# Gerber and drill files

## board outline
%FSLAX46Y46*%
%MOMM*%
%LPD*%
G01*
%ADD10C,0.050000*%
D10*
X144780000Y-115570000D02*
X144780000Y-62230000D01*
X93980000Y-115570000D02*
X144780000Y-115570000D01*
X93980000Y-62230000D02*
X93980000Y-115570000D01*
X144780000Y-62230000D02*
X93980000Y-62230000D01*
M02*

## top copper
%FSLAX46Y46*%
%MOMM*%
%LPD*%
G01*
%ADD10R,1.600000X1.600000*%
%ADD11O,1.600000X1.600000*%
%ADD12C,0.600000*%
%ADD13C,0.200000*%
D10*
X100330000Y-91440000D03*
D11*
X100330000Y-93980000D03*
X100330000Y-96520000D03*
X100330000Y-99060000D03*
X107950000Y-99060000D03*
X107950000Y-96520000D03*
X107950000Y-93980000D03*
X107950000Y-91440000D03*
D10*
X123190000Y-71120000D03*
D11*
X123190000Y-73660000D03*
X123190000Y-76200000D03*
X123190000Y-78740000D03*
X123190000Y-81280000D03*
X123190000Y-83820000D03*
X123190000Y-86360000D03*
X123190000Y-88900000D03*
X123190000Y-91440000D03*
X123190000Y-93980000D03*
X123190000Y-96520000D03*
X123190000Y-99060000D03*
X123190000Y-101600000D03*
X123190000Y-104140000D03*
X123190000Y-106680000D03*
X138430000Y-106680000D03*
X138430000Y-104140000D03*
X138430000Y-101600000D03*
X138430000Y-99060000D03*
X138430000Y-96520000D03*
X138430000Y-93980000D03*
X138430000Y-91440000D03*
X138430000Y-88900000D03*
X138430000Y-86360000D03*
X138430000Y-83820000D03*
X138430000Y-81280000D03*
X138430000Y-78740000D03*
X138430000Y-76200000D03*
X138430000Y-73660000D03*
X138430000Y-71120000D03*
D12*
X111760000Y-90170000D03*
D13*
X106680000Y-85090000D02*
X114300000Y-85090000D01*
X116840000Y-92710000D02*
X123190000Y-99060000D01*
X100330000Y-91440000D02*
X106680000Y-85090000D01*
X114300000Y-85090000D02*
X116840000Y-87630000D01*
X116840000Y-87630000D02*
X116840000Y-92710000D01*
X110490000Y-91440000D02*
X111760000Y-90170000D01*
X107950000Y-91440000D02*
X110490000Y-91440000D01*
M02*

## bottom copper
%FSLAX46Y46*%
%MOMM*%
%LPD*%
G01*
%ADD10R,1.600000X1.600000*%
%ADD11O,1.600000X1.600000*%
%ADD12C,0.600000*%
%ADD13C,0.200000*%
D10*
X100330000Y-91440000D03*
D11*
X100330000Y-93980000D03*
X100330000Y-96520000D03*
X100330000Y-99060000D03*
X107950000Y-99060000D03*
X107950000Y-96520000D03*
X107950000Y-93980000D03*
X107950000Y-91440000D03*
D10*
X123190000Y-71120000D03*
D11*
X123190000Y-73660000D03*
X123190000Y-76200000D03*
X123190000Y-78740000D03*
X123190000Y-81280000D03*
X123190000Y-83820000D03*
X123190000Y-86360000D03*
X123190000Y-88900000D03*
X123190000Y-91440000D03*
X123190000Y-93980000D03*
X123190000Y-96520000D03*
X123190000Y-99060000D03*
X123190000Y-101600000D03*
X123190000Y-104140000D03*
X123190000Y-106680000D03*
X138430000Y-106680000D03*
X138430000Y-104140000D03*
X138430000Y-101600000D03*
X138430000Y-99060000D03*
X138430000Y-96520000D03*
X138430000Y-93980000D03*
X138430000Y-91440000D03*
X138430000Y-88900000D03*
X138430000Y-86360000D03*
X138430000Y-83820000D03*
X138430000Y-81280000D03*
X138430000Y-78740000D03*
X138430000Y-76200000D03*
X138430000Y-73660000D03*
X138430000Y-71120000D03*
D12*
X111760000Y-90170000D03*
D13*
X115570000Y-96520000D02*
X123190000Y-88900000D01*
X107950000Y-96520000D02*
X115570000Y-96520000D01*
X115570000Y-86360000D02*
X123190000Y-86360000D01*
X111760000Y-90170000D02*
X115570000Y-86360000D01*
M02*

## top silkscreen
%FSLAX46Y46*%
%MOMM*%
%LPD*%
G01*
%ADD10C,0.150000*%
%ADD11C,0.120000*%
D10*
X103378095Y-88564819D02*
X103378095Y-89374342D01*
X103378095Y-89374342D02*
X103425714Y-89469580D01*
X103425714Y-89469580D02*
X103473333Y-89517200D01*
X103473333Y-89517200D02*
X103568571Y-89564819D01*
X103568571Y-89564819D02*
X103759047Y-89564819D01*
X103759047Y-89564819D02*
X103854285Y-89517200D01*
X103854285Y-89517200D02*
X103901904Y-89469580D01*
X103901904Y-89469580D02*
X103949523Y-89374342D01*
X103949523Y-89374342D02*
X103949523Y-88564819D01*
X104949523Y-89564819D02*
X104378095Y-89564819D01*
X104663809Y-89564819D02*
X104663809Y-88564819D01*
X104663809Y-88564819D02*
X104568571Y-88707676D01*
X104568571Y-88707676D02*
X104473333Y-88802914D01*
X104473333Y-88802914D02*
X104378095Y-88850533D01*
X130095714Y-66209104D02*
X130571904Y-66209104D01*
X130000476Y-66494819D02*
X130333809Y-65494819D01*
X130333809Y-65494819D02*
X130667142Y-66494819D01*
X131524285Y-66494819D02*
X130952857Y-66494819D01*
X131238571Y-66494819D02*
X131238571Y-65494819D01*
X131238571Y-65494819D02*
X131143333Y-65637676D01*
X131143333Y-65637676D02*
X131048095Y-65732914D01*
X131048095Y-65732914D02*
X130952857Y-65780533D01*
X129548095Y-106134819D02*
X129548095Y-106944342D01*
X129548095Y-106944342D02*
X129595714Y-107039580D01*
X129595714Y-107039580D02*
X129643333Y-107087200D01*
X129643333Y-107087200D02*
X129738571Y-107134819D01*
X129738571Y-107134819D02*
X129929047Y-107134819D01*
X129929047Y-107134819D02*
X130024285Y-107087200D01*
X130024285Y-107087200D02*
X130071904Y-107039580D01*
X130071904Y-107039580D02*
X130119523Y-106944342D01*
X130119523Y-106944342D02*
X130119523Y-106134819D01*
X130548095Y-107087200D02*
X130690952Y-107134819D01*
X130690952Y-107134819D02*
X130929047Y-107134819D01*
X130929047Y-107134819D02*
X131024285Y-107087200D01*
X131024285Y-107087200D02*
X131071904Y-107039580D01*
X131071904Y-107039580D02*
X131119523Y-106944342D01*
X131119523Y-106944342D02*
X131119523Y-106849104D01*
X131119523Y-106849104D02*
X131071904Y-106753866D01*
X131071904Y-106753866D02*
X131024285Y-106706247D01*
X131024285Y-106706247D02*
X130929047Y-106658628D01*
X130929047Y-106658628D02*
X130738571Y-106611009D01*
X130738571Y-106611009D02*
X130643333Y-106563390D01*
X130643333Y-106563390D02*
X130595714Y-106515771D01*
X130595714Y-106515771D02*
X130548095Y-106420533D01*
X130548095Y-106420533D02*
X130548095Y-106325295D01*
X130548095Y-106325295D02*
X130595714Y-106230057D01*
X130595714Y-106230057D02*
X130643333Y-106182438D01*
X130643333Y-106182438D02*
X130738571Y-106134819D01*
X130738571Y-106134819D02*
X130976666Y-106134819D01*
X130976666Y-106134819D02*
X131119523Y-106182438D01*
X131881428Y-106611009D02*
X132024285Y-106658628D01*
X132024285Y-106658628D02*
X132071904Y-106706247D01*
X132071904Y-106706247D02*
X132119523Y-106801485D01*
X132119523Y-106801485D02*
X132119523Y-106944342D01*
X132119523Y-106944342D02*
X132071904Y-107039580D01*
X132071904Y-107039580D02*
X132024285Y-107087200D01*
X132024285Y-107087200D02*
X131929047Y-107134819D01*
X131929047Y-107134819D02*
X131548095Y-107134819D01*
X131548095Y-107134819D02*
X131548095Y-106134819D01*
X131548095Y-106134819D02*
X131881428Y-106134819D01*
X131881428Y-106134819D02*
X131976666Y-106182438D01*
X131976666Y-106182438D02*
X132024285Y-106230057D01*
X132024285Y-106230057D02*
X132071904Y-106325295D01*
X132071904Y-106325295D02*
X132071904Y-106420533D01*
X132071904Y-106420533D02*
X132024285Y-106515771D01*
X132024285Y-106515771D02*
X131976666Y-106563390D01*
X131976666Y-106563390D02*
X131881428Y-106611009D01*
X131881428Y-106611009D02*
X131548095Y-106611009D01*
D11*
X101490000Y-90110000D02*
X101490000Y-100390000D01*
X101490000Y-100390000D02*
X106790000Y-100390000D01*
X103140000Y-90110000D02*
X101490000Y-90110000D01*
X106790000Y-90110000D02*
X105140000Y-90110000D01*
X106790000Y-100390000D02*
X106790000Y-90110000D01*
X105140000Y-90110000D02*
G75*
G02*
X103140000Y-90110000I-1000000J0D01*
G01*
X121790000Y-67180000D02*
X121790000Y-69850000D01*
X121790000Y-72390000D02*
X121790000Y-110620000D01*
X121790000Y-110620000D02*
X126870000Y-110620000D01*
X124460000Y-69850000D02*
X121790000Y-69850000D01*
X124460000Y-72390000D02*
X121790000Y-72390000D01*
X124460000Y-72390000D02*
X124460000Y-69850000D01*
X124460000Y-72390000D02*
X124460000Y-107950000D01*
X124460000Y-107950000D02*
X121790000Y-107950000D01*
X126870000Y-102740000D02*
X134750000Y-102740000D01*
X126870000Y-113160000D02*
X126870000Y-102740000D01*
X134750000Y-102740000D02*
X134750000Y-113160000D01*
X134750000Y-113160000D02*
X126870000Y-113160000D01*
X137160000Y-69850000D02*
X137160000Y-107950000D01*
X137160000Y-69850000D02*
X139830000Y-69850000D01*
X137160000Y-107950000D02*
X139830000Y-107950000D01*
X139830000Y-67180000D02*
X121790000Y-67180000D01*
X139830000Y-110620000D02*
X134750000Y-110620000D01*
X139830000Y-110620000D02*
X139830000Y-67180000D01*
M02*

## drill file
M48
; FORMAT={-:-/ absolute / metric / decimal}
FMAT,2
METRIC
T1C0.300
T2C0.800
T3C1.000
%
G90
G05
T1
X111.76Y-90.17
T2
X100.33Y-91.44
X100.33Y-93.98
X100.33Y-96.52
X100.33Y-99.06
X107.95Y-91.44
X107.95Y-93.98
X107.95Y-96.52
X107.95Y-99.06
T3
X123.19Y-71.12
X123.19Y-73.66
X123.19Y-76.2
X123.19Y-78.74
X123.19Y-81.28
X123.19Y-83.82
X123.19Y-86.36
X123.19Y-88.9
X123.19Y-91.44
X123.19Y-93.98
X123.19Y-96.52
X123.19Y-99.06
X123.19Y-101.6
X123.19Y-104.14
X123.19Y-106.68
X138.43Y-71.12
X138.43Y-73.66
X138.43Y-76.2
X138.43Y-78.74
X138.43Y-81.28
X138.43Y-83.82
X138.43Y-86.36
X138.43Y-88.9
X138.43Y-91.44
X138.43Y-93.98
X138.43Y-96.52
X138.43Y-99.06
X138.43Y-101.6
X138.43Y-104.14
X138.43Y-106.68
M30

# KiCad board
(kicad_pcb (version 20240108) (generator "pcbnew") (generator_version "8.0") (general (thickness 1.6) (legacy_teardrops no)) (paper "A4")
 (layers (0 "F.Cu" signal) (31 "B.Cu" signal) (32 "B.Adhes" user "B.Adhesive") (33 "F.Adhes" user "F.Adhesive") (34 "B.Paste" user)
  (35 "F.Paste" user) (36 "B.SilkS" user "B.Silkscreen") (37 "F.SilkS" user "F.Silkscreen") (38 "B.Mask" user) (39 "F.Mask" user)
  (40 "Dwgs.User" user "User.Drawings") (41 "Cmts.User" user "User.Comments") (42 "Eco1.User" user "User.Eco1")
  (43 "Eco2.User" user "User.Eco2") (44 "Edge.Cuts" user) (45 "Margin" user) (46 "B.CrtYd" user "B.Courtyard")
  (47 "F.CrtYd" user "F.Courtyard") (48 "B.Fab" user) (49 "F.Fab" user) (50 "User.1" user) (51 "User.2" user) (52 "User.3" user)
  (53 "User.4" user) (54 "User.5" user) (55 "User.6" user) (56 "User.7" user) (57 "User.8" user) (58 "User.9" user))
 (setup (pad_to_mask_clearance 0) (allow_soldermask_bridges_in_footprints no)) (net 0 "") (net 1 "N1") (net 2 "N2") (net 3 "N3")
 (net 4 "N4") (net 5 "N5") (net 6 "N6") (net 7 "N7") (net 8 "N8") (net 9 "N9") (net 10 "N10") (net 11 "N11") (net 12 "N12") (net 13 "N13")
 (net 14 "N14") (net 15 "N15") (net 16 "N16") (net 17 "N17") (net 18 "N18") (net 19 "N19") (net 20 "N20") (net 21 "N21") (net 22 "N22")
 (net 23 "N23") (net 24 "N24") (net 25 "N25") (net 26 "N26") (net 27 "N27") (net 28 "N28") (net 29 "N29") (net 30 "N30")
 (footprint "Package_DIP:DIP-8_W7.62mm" (layer "F.Cu") (at 100.33 91.44)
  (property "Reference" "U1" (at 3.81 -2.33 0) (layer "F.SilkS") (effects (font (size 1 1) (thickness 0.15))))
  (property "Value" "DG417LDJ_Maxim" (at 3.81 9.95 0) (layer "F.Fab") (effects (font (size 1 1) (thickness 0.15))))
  (fp_line (start 1.16 -1.33) (end 1.16 8.95) (stroke (width 0.12) (type solid)) (layer "F.SilkS"))
  (fp_line (start 1.16 8.95) (end 6.46 8.95) (stroke (width 0.12) (type solid)) (layer "F.SilkS"))
  (fp_line (start 2.81 -1.33) (end 1.16 -1.33) (stroke (width 0.12) (type solid)) (layer "F.SilkS"))
  (fp_line (start 6.46 -1.33) (end 4.81 -1.33) (stroke (width 0.12) (type solid)) (layer "F.SilkS"))
  (fp_line (start 6.46 8.95) (end 6.46 -1.33) (stroke (width 0.12) (type solid)) (layer "F.SilkS"))
  (fp_arc (start 4.81 -1.33) (mid 3.81 -0.33) (end 2.81 -1.33) (stroke (width 0.12) (type solid)) (layer "F.SilkS"))
  (pad "1" thru_hole rect (at 0 0) (size 1.6 1.6) (drill 0.8) (layers "*.Cu" "*.Mask") (remove_unused_layers no) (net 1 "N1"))
  (pad "2" thru_hole oval (at 0 2.54) (size 1.6 1.6) (drill 0.8) (layers "*.Cu" "*.Mask") (remove_unused_layers no))
  (pad "3" thru_hole oval (at 0 5.08) (size 1.6 1.6) (drill 0.8) (layers "*.Cu" "*.Mask") (remove_unused_layers no))
  (pad "4" thru_hole oval (at 0 7.62) (size 1.6 1.6) (drill 0.8) (layers "*.Cu" "*.Mask") (remove_unused_layers no))
  (pad "5" thru_hole oval (at 7.62 7.62) (size 1.6 1.6) (drill 0.8) (layers "*.Cu" "*.Mask") (remove_unused_layers no))
  (pad "6" thru_hole oval (at 7.62 5.08) (size 1.6 1.6) (drill 0.8) (layers "*.Cu" "*.Mask") (remove_unused_layers no) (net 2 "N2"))
  (pad "7" thru_hole oval (at 7.62 2.54) (size 1.6 1.6) (drill 0.8) (layers "*.Cu" "*.Mask") (remove_unused_layers no))
  (pad "8" thru_hole oval (at 7.62 0) (size 1.6 1.6) (drill 0.8) (layers "*.Cu" "*.Mask") (remove_unused_layers no) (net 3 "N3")))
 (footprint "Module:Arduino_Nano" (layer "F.Cu") (at 123.19 71.12)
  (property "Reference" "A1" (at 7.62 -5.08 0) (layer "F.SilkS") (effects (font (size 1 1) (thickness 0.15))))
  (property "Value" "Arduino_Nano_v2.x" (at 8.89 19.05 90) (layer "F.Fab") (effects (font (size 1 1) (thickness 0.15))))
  (fp_line (start -1.4 -3.94) (end -1.4 -1.27) (stroke (width 0.12) (type solid)) (layer "F.SilkS"))
  (fp_line (start -1.4 1.27) (end -1.4 39.5) (stroke (width 0.12) (type solid)) (layer "F.SilkS"))
  (fp_line (start -1.4 39.5) (end 3.68 39.5) (stroke (width 0.12) (type solid)) (layer "F.SilkS"))
  (fp_line (start 1.27 -1.27) (end -1.4 -1.27) (stroke (width 0.12) (type solid)) (layer "F.SilkS"))
  (fp_line (start 1.27 1.27) (end -1.4 1.27) (stroke (width 0.12) (type solid)) (layer "F.SilkS"))
  (fp_line (start 1.27 1.27) (end 1.27 -1.27) (stroke (width 0.12) (type solid)) (layer "F.SilkS"))
  (fp_line (start 1.27 1.27) (end 1.27 36.83) (stroke (width 0.12) (type solid)) (layer "F.SilkS"))
  (fp_line (start 1.27 36.83) (end -1.4 36.83) (stroke (width 0.12) (type solid)) (layer "F.SilkS"))
  (fp_line (start 3.68 31.62) (end 11.56 31.62) (stroke (width 0.12) (type solid)) (layer "F.SilkS"))
  (fp_line (start 3.68 42.04) (end 3.68 31.62) (stroke (width 0.12) (type solid)) (layer "F.SilkS"))
  (fp_line (start 11.56 31.62) (end 11.56 42.04) (stroke (width 0.12) (type solid)) (layer "F.SilkS"))
  (fp_line (start 11.56 42.04) (end 3.68 42.04) (stroke (width 0.12) (type solid)) (layer "F.SilkS"))
  (fp_line (start 13.97 -1.27) (end 13.97 36.83) (stroke (width 0.12) (type solid)) (layer "F.SilkS"))
  (fp_line (start 13.97 -1.27) (end 16.64 -1.27) (stroke (width 0.12) (type solid)) (layer "F.SilkS"))
  (fp_line (start 13.97 36.83) (end 16.64 36.83) (stroke (width 0.12) (type solid)) (layer "F.SilkS"))
  (fp_line (start 16.64 -3.94) (end -1.4 -3.94) (stroke (width 0.12) (type solid)) (layer "F.SilkS"))
  (fp_line (start 16.64 39.5) (end 11.56 39.5) (stroke (width 0.12) (type solid)) (layer "F.SilkS"))
  (fp_line (start 16.64 39.5) (end 16.64 -3.94) (stroke (width 0.12) (type solid)) (layer "F.SilkS"))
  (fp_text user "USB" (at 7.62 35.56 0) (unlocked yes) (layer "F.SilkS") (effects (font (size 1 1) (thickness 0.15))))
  (pad "1" thru_hole rect (at 0 0) (size 1.6 1.6) (drill 1) (layers "*.Cu" "*.Mask") (remove_unused_layers no) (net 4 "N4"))
  (pad "2" thru_hole oval (at 0 2.54) (size 1.6 1.6) (drill 1) (layers "*.Cu" "*.Mask") (remove_unused_layers no) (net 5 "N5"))
  (pad "3" thru_hole oval (at 0 5.08) (size 1.6 1.6) (drill 1) (layers "*.Cu" "*.Mask") (remove_unused_layers no) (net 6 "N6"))
  (pad "4" thru_hole oval (at 0 7.62) (size 1.6 1.6) (drill 1) (layers "*.Cu" "*.Mask") (remove_unused_layers no) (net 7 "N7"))
  (pad "5" thru_hole oval (at 0 10.16) (size 1.6 1.6) (drill 1) (layers "*.Cu" "*.Mask") (remove_unused_layers no) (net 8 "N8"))
  (pad "6" thru_hole oval (at 0 12.7) (size 1.6 1.6) (drill 1) (layers "*.Cu" "*.Mask") (remove_unused_layers no) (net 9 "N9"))
  (pad "7" thru_hole oval (at 0 15.24) (size 1.6 1.6) (drill 1) (layers "*.Cu" "*.Mask") (remove_unused_layers no) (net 3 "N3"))
  (pad "8" thru_hole oval (at 0 17.78) (size 1.6 1.6) (drill 1) (layers "*.Cu" "*.Mask") (remove_unused_layers no) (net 2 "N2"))
  (pad "9" thru_hole oval (at 0 20.32) (size 1.6 1.6) (drill 1) (layers "*.Cu" "*.Mask") (remove_unused_layers no) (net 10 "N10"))
  (pad "10" thru_hole oval (at 0 22.86) (size 1.6 1.6) (drill 1) (layers "*.Cu" "*.Mask") (remove_unused_layers no) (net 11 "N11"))
  (pad "11" thru_hole oval (at 0 25.4) (size 1.6 1.6) (drill 1) (layers "*.Cu" "*.Mask") (remove_unused_layers no) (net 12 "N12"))
  (pad "12" thru_hole oval (at 0 27.94) (size 1.6 1.6) (drill 1) (layers "*.Cu" "*.Mask") (remove_unused_layers no) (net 1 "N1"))
  (pad "13" thru_hole oval (at 0 30.48) (size 1.6 1.6) (drill 1) (layers "*.Cu" "*.Mask") (remove_unused_layers no) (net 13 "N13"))
  (pad "14" thru_hole oval (at 0 33.02) (size 1.6 1.6) (drill 1) (layers "*.Cu" "*.Mask") (remove_unused_layers no) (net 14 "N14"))
  (pad "15" thru_hole oval (at 0 35.56) (size 1.6 1.6) (drill 1) (layers "*.Cu" "*.Mask") (remove_unused_layers no) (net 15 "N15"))
  (pad "16" thru_hole oval (at 15.24 35.56) (size 1.6 1.6) (drill 1) (layers "*.Cu" "*.Mask") (remove_unused_layers no) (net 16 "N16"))
  (pad "17" thru_hole oval (at 15.24 33.02) (size 1.6 1.6) (drill 1) (layers "*.Cu" "*.Mask") (remove_unused_layers no) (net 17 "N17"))
  (pad "18" thru_hole oval (at 15.24 30.48) (size 1.6 1.6) (drill 1) (layers "*.Cu" "*.Mask") (remove_unused_layers no) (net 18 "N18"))
  (pad "19" thru_hole oval (at 15.24 27.94) (size 1.6 1.6) (drill 1) (layers "*.Cu" "*.Mask") (remove_unused_layers no) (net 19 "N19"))
  (pad "20" thru_hole oval (at 15.24 25.4) (size 1.6 1.6) (drill 1) (layers "*.Cu" "*.Mask") (remove_unused_layers no) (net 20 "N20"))
  (pad "21" thru_hole oval (at 15.24 22.86) (size 1.6 1.6) (drill 1) (layers "*.Cu" "*.Mask") (remove_unused_layers no) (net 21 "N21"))
  (pad "22" thru_hole oval (at 15.24 20.32) (size 1.6 1.6) (drill 1) (layers "*.Cu" "*.Mask") (remove_unused_layers no) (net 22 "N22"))
  (pad "23" thru_hole oval (at 15.24 17.78) (size 1.6 1.6) (drill 1) (layers "*.Cu" "*.Mask") (remove_unused_layers no) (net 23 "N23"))
  (pad "24" thru_hole oval (at 15.24 15.24) (size 1.6 1.6) (drill 1) (layers "*.Cu" "*.Mask") (remove_unused_layers no) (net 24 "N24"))
  (pad "25" thru_hole oval (at 15.24 12.7) (size 1.6 1.6) (drill 1) (layers "*.Cu" "*.Mask") (remove_unused_layers no) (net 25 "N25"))
  (pad "26" thru_hole oval (at 15.24 10.16) (size 1.6 1.6) (drill 1) (layers "*.Cu" "*.Mask") (remove_unused_layers no) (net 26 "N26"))
  (pad "27" thru_hole oval (at 15.24 7.62) (size 1.6 1.6) (drill 1) (layers "*.Cu" "*.Mask") (remove_unused_layers no) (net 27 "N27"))
  (pad "28" thru_hole oval (at 15.24 5.08) (size 1.6 1.6) (drill 1) (layers "*.Cu" "*.Mask") (remove_unused_layers no) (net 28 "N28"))
  (pad "29" thru_hole oval (at 15.24 2.54) (size 1.6 1.6) (drill 1) (layers "*.Cu" "*.Mask") (remove_unused_layers no) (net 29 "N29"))
  (pad "30" thru_hole oval (at 15.24 0) (size 1.6 1.6) (drill 1) (layers "*.Cu" "*.Mask") (remove_unused_layers no) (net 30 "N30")))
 (gr_line (start 144.78 115.57) (end 144.78 62.23) (stroke (width 0.05) (type default)) (layer "Edge.Cuts"))
 (gr_line (start 93.98 115.57) (end 144.78 115.57) (stroke (width 0.05) (type default)) (layer "Edge.Cuts"))
 (gr_line (start 93.98 62.23) (end 93.98 115.57) (stroke (width 0.05) (type default)) (layer "Edge.Cuts"))
 (gr_line (start 144.78 62.23) (end 93.98 62.23) (stroke (width 0.05) (type default)) (layer "Edge.Cuts"))
 (segment (start 115.57 96.52) (end 123.19 88.9) (width 0.2) (layer "B.Cu") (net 2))
 (segment (start 107.95 96.52) (end 115.57 96.52) (width 0.2) (layer "B.Cu") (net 2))
 (segment (start 106.68 85.09) (end 114.3 85.09) (width 0.2) (layer "F.Cu") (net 1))
 (segment (start 116.84 92.71) (end 123.19 99.06) (width 0.2) (layer "F.Cu") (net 1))
 (segment (start 100.33 91.44) (end 106.68 85.09) (width 0.2) (layer "F.Cu") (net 1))
 (segment (start 114.3 85.09) (end 116.84 87.63) (width 0.2) (layer "F.Cu") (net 1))
 (segment (start 116.84 87.63) (end 116.84 92.71) (width 0.2) (layer "F.Cu") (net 1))
 (segment (start 110.49 91.44) (end 111.76 90.17) (width 0.2) (layer "F.Cu") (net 3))
 (segment (start 107.95 91.44) (end 110.49 91.44) (width 0.2) (layer "F.Cu") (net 3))
 (via (at 111.76 90.17) (size 0.6) (drill 0.3) (layers "F.Cu" "B.Cu") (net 3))
 (segment (start 115.57 86.36) (end 123.19 86.36) (width 0.2) (layer "B.Cu") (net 3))
 (segment (start 111.76 90.17) (end 115.57 86.36) (width 0.2) (layer "B.Cu") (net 3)))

